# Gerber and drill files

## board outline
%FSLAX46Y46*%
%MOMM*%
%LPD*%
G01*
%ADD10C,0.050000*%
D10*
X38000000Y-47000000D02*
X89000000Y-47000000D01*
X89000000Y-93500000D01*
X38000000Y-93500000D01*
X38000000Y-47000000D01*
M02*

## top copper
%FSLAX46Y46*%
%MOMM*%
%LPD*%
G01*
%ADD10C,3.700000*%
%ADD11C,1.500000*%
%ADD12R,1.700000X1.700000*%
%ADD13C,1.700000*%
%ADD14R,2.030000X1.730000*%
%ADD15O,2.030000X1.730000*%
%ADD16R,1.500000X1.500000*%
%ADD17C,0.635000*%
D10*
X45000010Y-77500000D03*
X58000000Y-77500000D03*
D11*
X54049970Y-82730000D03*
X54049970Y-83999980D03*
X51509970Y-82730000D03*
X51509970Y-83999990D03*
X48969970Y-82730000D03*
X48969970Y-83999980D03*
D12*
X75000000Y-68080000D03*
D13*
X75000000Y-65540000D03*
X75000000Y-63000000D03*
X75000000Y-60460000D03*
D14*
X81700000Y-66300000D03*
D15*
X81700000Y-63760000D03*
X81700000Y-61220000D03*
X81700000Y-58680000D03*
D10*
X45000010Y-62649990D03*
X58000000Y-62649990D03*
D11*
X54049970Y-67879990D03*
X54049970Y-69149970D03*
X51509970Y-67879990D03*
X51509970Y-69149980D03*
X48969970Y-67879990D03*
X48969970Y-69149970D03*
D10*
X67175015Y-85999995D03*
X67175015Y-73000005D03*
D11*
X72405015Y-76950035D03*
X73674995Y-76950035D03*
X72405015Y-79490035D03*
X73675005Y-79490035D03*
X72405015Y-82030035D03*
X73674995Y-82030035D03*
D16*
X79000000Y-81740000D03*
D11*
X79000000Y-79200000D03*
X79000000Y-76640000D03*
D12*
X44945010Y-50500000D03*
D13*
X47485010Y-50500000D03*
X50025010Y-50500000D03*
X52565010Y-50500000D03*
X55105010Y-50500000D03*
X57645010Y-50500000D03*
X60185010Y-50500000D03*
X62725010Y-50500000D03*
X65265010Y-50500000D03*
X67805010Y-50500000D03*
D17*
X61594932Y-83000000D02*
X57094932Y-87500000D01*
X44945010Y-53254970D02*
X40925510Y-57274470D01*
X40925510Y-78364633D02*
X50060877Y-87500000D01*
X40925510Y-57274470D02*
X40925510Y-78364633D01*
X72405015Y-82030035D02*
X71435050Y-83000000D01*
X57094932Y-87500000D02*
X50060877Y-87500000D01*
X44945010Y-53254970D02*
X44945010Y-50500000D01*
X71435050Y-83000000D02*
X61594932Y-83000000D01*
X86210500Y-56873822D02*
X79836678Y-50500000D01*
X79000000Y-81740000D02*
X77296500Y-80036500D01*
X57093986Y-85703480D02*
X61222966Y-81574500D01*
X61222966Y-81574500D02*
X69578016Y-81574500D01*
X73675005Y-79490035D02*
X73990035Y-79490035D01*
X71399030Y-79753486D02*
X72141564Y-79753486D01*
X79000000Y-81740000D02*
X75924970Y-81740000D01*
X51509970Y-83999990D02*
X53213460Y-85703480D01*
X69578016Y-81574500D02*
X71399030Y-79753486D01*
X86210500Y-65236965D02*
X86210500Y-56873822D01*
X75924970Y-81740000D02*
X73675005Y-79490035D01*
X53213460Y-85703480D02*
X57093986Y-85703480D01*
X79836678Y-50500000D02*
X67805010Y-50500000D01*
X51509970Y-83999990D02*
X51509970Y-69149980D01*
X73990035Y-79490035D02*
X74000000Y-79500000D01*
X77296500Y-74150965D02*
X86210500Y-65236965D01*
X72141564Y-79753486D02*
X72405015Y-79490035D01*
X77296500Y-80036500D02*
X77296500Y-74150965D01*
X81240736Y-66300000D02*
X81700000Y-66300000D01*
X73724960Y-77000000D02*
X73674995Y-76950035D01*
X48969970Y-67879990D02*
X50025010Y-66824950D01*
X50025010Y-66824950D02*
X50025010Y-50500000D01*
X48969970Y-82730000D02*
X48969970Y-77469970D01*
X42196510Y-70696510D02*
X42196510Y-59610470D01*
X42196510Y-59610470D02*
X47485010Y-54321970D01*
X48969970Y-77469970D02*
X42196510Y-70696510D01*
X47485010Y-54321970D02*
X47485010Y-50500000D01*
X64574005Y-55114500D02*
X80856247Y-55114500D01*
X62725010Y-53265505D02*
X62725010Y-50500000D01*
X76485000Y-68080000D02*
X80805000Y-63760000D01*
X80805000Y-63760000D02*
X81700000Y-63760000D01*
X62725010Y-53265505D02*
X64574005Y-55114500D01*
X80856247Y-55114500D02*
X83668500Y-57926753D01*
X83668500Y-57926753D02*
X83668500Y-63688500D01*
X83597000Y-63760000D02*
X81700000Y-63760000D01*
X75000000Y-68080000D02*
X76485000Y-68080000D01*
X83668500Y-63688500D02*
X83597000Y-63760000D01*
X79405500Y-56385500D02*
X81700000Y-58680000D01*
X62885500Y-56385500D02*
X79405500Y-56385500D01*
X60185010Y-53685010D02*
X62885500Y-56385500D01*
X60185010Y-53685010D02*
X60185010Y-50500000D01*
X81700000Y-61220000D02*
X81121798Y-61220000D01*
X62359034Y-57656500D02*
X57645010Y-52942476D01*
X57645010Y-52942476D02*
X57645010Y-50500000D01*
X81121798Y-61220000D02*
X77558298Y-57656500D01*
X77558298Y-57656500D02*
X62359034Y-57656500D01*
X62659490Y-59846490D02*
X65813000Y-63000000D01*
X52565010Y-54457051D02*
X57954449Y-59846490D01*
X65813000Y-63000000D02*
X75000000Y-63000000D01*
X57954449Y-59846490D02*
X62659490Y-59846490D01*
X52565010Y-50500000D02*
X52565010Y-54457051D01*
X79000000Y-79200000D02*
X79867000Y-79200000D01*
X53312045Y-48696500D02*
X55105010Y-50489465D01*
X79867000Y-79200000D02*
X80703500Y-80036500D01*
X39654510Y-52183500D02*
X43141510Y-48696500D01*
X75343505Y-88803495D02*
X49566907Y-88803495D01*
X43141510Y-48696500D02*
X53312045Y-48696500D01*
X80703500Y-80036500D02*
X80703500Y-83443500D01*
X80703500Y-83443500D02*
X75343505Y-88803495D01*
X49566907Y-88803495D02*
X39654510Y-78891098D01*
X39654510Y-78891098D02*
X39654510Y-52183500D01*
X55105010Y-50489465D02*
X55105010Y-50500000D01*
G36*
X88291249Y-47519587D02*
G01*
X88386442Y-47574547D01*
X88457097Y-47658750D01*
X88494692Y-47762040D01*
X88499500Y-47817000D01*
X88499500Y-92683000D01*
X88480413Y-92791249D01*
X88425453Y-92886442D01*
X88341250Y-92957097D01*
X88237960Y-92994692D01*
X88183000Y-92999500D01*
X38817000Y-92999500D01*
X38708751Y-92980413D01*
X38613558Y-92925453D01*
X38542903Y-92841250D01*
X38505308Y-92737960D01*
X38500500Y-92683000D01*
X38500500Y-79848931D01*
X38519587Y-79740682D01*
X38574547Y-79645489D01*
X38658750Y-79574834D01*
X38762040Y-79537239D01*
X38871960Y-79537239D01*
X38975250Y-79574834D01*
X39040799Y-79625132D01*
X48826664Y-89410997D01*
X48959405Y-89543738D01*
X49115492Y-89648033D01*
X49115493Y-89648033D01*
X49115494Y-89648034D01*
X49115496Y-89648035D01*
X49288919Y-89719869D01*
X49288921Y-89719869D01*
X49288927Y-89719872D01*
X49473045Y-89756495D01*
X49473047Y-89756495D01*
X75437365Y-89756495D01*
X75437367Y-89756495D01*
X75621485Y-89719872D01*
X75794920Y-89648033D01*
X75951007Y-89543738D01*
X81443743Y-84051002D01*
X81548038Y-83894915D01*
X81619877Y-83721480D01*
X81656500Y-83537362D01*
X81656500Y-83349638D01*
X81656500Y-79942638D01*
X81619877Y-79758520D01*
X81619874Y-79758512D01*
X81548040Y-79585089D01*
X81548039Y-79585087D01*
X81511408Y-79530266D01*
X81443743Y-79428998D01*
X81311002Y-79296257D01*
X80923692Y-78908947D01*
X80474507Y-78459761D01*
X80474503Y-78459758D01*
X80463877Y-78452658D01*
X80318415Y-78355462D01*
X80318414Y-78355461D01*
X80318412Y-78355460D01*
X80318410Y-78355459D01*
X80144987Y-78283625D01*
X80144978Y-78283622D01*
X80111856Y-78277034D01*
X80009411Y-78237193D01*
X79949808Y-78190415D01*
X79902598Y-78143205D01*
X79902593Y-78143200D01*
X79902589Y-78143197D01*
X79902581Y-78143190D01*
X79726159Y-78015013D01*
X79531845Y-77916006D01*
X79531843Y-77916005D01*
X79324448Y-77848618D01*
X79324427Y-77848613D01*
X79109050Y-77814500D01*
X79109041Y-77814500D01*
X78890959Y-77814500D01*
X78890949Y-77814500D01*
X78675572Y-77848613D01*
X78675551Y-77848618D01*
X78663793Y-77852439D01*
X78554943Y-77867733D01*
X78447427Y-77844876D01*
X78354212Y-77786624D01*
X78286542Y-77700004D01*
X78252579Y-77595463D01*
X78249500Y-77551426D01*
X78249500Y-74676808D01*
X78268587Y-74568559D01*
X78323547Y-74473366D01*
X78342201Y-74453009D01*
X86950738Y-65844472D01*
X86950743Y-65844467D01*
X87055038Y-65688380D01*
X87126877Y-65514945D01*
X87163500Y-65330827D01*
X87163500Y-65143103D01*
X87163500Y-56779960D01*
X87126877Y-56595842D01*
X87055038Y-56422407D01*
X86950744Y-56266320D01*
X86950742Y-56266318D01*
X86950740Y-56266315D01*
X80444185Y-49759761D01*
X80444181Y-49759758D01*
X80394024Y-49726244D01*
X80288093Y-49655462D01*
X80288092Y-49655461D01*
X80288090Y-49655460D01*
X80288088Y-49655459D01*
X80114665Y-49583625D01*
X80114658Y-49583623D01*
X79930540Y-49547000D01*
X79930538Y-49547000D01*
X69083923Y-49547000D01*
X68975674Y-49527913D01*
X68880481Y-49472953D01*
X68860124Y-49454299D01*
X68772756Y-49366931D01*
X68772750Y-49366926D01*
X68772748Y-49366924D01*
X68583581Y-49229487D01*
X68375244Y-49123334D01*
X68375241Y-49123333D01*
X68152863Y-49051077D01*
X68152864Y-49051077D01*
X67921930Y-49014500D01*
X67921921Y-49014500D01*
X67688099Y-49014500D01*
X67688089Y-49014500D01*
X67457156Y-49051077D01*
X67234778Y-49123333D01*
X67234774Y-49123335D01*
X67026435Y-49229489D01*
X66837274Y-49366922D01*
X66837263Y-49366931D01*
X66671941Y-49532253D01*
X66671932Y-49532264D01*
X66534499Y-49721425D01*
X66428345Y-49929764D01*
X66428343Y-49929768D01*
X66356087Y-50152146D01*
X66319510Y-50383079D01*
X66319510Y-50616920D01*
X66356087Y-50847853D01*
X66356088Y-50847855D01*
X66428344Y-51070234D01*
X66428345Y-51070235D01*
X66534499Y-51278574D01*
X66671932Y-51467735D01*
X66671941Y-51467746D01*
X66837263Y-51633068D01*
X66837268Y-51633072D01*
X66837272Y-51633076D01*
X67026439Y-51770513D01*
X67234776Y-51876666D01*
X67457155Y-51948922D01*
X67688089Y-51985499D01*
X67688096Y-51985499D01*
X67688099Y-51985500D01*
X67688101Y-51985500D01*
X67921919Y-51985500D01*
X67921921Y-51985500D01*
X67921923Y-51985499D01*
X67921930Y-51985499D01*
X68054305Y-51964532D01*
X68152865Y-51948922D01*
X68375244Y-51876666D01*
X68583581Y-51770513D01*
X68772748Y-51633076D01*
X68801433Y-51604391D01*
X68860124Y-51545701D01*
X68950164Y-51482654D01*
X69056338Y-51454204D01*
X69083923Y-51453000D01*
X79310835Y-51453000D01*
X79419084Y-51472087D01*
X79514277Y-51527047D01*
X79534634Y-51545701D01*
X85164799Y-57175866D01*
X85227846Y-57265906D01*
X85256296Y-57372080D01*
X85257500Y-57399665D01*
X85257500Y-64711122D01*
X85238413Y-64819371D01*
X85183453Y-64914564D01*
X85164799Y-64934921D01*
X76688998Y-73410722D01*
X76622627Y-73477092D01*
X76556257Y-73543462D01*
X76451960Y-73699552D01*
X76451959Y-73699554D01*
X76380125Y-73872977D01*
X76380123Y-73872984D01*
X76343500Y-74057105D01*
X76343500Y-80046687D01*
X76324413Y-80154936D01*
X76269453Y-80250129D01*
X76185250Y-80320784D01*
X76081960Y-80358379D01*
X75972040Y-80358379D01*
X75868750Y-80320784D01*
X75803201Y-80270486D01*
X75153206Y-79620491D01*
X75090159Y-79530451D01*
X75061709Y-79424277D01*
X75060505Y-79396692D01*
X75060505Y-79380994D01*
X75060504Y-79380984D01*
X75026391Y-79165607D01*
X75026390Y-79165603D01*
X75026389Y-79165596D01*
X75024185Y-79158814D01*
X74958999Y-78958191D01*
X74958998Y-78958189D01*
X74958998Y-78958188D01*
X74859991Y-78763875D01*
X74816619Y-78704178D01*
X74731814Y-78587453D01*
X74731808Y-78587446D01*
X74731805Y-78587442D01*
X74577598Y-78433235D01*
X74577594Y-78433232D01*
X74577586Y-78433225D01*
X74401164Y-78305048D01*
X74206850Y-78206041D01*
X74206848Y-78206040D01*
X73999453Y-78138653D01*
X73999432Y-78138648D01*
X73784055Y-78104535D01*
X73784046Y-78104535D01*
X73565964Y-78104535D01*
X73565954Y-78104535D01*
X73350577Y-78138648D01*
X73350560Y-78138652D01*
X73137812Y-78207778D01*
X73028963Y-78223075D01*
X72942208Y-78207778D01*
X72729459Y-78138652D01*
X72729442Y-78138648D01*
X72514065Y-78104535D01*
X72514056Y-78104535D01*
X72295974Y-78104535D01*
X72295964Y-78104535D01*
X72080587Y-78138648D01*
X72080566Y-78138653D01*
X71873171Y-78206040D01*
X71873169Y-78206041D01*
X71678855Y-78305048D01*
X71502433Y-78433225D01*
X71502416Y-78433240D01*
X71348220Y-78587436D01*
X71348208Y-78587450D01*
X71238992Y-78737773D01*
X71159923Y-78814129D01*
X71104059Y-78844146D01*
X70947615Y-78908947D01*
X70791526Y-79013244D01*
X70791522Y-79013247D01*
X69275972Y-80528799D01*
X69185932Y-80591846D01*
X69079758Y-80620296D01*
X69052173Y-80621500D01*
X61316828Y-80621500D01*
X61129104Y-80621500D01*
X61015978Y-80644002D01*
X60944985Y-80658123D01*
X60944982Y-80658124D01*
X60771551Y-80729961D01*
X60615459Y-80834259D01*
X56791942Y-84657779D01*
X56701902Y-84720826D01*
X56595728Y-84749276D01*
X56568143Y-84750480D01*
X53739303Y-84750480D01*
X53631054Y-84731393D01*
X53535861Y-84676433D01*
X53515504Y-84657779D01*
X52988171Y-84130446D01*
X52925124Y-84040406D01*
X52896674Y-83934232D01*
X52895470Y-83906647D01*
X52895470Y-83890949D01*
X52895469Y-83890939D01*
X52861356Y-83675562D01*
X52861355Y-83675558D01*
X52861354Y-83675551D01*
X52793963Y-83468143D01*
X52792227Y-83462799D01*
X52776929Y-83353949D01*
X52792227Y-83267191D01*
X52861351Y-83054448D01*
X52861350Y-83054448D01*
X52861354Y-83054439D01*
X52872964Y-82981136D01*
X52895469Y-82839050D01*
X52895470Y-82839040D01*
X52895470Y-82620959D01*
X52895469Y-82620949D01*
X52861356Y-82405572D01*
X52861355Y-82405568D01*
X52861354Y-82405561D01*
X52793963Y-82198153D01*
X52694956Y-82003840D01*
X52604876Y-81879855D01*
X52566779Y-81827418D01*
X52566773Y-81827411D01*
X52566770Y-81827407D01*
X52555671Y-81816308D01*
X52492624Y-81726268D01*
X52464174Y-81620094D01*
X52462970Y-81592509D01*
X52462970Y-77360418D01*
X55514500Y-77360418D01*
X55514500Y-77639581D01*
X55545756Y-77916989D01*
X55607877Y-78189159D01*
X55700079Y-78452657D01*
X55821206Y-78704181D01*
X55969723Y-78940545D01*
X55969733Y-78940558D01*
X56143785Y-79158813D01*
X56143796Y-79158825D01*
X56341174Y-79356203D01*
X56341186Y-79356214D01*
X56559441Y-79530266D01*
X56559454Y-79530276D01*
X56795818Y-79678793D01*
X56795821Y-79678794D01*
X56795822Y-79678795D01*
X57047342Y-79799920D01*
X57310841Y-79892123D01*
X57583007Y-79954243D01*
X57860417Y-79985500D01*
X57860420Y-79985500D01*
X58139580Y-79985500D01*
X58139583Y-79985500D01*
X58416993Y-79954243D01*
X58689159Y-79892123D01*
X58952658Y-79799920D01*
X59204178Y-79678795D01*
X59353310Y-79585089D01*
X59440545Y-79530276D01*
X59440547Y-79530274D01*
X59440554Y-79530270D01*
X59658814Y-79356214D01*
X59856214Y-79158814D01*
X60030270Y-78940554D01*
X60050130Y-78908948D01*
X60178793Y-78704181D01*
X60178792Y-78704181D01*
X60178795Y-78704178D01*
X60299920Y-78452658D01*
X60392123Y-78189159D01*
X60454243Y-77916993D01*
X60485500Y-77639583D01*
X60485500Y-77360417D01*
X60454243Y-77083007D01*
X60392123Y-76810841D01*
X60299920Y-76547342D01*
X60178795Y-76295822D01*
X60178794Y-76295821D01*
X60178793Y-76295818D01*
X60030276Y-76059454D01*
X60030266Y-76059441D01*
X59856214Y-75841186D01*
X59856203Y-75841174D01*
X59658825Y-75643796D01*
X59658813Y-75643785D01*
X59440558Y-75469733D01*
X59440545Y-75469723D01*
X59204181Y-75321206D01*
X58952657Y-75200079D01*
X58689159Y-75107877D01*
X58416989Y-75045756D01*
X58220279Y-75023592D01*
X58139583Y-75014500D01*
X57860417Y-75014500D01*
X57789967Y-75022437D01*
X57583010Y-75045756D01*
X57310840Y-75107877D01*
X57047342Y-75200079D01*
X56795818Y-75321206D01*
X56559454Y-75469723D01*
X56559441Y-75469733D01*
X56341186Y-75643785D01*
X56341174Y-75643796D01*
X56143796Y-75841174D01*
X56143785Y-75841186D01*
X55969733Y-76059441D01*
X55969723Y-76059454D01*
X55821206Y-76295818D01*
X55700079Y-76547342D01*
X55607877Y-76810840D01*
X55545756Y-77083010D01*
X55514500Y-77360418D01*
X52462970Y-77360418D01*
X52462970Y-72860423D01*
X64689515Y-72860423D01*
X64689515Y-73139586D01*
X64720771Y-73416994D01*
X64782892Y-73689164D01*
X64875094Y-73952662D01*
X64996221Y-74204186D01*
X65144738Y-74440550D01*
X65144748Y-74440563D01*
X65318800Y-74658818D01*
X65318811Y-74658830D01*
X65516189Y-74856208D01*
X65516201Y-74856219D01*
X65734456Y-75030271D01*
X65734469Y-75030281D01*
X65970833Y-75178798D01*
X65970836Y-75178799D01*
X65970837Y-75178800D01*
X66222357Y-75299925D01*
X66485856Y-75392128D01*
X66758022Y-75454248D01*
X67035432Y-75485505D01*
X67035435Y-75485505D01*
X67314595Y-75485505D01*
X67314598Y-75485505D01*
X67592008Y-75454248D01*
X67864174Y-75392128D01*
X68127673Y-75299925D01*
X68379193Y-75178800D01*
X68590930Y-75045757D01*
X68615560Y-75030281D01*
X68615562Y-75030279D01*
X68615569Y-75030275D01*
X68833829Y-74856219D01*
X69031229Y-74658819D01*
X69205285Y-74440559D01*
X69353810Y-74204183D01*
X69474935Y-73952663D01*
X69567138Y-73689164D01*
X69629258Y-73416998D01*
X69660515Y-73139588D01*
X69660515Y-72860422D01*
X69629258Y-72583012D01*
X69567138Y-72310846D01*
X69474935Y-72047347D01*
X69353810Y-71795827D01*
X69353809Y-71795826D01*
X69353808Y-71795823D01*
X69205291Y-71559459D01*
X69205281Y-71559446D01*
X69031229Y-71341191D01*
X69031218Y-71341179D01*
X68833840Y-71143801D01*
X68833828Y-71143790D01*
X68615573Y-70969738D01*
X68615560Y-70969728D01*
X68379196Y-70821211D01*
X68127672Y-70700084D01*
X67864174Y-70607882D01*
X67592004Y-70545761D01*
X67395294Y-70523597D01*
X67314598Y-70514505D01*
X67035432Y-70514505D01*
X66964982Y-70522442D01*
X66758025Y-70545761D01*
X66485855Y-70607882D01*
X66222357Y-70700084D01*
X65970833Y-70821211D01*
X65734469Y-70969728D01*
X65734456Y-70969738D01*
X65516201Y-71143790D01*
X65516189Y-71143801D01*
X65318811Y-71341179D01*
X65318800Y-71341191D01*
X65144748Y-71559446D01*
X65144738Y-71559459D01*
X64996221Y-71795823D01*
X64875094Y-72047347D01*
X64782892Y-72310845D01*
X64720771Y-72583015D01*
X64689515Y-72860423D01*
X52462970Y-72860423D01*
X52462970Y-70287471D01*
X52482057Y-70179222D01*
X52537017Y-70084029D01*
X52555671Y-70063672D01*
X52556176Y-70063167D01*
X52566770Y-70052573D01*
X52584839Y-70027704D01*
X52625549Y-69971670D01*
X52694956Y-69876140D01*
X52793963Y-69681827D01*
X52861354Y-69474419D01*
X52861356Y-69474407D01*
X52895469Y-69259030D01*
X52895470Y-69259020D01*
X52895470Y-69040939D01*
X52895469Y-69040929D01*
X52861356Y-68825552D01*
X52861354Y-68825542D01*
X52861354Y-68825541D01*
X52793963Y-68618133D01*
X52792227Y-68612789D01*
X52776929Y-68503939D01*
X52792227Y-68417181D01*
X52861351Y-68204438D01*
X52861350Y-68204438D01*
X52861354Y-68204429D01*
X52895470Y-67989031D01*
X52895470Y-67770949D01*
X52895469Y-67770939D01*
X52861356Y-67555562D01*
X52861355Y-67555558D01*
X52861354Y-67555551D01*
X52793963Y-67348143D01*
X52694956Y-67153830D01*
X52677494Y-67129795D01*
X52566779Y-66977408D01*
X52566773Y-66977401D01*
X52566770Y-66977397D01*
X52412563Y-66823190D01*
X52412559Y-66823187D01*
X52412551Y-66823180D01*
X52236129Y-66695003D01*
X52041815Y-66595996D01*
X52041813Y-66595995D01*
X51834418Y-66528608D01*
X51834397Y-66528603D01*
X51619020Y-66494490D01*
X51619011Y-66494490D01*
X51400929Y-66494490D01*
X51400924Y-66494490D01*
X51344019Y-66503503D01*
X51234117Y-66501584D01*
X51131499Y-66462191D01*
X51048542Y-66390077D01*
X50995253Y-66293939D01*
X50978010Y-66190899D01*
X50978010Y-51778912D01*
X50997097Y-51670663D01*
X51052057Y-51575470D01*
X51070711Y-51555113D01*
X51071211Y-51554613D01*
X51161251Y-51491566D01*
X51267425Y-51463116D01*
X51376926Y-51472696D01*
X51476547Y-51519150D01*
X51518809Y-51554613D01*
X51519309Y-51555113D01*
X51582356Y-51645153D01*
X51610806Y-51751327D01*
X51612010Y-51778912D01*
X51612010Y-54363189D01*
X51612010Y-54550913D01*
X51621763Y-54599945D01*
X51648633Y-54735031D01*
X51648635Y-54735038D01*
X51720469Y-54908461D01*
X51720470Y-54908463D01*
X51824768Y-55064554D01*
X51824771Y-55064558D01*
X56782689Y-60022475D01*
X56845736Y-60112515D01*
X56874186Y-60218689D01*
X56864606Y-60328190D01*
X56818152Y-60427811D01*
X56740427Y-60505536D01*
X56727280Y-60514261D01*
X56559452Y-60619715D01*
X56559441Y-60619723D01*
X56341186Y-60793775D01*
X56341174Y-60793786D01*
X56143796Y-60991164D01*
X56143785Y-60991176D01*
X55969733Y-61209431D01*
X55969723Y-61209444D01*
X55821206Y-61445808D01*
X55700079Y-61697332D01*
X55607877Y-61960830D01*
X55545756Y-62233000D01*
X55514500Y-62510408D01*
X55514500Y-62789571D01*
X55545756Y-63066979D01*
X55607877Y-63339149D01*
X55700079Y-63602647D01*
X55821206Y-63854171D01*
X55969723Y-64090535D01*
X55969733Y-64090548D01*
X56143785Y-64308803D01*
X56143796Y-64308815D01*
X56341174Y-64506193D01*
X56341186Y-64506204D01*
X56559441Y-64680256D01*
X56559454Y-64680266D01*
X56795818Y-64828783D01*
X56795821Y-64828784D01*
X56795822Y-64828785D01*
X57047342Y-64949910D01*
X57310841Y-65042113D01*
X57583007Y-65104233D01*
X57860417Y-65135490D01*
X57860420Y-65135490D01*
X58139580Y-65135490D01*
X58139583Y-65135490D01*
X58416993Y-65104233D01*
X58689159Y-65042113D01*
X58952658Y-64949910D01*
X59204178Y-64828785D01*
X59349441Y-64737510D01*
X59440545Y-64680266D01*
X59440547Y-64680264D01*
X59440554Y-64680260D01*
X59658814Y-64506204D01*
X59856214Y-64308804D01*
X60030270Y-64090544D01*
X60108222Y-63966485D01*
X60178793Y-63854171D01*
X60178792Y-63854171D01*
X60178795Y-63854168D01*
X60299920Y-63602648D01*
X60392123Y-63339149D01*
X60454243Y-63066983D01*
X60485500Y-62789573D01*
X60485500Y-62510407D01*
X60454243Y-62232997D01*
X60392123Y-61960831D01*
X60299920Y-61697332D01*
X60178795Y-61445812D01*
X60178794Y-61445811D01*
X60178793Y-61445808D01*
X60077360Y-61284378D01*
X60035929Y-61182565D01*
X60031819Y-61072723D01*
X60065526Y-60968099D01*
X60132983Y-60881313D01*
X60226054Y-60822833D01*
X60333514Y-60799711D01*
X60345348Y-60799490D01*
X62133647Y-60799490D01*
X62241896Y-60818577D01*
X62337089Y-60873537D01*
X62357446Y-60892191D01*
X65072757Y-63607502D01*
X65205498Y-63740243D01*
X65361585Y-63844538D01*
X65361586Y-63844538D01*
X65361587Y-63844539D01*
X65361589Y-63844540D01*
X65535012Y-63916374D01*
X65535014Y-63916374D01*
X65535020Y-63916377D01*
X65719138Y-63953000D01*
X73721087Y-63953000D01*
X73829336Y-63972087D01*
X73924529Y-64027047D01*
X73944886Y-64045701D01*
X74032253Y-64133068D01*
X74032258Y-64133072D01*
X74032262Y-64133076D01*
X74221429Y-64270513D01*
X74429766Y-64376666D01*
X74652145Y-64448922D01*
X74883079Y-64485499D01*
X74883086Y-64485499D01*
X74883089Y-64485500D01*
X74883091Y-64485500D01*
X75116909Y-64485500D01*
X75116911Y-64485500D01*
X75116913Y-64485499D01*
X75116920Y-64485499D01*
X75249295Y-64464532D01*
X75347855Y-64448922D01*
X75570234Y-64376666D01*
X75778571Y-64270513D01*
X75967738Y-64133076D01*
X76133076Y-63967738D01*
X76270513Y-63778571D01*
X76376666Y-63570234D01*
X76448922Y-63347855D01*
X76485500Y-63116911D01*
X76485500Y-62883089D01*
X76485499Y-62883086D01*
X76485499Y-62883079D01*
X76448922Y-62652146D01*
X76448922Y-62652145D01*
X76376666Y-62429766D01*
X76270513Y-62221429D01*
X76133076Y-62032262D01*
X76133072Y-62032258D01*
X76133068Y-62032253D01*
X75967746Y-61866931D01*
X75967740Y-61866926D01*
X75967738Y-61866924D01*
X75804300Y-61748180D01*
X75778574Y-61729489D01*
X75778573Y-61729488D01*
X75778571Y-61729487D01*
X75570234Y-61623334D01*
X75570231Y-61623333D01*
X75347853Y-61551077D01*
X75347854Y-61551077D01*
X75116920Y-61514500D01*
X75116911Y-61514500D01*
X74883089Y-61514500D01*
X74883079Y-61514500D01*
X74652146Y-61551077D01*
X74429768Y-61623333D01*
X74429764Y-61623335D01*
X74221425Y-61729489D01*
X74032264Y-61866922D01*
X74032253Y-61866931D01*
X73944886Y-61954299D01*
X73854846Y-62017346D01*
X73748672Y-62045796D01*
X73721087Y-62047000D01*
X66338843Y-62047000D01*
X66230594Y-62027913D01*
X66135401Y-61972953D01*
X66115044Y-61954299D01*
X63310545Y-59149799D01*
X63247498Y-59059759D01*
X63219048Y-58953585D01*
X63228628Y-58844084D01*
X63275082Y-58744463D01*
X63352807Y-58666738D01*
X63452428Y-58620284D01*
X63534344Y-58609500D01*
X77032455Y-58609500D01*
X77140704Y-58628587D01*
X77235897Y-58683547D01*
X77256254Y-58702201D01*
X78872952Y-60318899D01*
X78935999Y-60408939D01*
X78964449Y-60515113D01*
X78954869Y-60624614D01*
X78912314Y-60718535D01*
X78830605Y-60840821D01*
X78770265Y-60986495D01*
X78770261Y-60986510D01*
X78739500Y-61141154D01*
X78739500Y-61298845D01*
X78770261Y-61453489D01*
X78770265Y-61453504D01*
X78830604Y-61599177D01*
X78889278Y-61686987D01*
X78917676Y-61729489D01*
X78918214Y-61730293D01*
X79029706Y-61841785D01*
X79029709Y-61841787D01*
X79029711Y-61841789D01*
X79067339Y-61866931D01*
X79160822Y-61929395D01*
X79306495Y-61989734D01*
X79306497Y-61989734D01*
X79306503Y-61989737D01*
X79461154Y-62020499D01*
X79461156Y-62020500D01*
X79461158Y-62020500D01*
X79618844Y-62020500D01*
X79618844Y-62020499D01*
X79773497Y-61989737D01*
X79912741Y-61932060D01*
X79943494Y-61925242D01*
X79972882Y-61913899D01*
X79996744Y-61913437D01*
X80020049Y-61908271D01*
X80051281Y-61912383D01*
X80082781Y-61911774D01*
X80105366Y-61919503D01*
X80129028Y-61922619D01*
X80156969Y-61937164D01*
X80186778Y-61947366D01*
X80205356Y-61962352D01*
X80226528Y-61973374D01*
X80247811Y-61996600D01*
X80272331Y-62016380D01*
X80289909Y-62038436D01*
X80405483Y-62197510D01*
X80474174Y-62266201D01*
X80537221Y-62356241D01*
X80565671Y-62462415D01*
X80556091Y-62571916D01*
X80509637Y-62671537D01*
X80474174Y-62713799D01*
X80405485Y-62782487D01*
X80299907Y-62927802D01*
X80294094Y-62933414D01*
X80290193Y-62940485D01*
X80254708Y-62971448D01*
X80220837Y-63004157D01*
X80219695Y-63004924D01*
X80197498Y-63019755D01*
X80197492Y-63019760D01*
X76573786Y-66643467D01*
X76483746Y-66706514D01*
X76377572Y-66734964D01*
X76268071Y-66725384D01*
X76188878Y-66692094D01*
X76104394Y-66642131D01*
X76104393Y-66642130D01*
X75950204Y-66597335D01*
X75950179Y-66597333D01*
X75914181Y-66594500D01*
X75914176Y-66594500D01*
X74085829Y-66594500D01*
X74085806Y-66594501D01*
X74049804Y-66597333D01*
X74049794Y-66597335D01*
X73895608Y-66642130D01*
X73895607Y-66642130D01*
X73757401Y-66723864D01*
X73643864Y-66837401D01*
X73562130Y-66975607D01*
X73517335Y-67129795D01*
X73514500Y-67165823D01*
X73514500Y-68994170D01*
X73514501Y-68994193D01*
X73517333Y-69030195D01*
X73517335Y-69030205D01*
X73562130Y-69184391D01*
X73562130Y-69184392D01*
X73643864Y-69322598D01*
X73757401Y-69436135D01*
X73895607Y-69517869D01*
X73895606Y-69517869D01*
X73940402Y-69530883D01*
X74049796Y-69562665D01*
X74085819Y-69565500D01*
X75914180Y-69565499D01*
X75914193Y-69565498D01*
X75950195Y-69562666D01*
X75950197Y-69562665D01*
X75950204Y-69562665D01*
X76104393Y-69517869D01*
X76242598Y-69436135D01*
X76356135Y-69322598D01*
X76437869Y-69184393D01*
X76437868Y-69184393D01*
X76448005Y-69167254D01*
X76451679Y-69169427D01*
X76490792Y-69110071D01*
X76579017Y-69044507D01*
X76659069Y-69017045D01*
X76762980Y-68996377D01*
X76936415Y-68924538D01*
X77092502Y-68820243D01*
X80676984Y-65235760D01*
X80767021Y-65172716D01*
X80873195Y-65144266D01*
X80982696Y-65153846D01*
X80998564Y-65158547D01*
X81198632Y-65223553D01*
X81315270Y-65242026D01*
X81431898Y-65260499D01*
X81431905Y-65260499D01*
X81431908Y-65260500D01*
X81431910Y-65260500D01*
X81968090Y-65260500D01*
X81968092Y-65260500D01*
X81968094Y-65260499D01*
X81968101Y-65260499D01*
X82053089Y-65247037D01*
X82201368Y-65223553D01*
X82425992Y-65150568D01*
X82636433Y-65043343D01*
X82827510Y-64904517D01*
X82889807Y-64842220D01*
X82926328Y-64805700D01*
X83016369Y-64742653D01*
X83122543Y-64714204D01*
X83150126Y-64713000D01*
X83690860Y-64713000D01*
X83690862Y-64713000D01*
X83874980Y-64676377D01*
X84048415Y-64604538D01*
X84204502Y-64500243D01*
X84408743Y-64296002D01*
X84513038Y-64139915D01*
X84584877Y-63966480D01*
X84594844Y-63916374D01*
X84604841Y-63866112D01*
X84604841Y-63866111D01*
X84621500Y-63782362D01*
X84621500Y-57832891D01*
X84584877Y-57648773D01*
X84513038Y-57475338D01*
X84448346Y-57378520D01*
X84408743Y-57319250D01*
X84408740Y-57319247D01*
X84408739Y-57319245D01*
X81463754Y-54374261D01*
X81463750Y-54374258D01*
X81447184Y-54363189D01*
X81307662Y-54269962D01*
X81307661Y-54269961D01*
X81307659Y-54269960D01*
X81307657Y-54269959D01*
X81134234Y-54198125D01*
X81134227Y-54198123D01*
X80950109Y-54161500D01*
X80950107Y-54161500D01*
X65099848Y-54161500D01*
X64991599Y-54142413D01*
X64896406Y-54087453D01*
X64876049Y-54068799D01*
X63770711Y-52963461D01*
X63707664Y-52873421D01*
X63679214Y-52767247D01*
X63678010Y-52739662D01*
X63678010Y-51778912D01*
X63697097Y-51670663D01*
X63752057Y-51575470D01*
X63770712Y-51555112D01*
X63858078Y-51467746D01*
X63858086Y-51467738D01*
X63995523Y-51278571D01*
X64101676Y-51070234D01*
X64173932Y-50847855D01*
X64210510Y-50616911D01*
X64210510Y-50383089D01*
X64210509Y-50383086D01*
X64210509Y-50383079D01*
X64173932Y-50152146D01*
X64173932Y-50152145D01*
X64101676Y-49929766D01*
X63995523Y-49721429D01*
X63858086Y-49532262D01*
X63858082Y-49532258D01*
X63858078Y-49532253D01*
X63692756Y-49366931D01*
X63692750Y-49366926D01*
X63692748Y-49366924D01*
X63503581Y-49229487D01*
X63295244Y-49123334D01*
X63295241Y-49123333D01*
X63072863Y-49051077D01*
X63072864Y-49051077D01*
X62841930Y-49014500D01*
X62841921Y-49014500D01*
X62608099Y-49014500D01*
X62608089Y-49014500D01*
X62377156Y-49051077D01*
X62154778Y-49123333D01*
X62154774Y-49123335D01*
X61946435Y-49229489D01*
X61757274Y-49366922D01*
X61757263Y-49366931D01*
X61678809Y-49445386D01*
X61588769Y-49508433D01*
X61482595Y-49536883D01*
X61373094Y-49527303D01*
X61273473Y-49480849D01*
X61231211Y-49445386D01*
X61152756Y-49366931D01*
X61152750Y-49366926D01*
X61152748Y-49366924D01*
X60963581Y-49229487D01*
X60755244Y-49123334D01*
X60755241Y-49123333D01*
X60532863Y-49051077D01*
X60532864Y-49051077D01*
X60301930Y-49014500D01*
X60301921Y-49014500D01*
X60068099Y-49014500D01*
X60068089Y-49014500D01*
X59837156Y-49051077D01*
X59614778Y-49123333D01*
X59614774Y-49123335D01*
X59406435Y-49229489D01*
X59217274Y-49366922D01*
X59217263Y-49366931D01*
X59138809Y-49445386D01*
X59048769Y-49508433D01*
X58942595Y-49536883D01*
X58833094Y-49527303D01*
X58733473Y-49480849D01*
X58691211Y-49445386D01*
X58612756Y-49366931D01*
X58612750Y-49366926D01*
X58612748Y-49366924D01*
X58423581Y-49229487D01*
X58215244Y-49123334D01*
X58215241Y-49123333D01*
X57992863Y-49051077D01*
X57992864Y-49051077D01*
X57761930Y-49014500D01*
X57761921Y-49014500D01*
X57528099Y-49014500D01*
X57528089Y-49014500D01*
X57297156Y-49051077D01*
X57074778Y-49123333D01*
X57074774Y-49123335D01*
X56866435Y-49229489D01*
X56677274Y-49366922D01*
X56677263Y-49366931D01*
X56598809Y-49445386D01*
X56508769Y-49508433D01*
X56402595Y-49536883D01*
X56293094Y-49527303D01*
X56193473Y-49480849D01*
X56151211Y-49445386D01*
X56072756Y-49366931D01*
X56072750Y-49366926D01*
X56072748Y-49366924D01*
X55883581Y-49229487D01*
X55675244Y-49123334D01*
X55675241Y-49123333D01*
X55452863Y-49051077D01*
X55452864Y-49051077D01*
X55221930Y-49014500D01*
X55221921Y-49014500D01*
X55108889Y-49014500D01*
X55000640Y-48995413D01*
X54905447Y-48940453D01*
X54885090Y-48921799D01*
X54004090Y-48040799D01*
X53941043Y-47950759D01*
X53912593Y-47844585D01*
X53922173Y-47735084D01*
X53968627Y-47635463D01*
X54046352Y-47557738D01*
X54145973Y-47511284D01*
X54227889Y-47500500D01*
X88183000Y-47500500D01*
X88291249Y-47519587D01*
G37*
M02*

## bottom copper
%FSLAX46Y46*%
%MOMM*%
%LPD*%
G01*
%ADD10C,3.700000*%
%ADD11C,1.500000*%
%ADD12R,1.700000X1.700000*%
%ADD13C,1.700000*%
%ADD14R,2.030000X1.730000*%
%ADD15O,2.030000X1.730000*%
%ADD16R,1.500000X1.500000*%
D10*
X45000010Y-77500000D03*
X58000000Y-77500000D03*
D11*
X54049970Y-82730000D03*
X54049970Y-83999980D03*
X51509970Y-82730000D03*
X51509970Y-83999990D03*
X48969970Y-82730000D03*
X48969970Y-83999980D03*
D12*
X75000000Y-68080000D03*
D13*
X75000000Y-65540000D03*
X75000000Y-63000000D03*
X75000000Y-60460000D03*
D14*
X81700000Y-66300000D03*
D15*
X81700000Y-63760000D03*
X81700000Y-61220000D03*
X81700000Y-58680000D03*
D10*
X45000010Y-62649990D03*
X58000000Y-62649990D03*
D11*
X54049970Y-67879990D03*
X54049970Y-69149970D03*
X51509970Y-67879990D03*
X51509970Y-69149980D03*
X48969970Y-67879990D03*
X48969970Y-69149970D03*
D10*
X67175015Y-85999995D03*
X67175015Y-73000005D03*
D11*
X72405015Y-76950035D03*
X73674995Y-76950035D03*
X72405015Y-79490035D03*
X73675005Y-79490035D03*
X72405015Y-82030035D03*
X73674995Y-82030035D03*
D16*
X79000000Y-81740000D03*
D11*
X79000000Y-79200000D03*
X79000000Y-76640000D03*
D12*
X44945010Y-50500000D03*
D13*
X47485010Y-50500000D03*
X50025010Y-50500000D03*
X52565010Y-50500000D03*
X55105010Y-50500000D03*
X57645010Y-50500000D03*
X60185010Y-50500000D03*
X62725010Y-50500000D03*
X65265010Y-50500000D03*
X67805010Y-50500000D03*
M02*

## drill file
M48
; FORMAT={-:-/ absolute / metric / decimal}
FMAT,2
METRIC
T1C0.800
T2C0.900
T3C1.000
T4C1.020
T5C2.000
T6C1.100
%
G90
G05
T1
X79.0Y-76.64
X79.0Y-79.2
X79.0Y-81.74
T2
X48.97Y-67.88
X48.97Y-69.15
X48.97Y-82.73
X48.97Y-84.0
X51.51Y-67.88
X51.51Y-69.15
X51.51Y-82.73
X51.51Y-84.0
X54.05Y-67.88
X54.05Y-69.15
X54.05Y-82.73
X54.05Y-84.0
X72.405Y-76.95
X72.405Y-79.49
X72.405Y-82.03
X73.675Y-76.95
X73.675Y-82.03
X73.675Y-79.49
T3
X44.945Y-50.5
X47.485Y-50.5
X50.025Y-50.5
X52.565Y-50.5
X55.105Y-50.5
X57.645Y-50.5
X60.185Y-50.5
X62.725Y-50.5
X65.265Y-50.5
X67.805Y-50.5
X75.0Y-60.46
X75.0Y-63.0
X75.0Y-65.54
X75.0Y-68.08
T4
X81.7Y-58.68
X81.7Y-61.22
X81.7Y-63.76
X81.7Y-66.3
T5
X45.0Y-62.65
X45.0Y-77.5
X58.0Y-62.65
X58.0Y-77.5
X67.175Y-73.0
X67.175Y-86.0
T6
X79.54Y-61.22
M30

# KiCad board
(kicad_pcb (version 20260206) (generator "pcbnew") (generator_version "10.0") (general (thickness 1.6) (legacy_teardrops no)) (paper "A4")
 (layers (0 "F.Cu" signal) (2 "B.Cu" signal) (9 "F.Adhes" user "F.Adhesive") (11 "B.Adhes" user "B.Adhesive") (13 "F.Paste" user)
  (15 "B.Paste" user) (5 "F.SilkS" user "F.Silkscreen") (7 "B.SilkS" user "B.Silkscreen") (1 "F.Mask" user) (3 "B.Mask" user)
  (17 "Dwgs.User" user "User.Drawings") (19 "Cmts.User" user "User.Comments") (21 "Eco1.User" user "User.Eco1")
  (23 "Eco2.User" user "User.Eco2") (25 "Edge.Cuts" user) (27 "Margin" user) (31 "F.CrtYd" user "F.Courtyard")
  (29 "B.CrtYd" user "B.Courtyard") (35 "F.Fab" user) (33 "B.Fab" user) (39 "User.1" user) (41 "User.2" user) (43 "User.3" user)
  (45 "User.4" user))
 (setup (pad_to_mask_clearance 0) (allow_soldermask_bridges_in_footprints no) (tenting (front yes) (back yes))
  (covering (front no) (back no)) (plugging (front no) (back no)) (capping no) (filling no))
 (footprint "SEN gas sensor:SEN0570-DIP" (layer "F.Cu") (at 45.00001 77.5)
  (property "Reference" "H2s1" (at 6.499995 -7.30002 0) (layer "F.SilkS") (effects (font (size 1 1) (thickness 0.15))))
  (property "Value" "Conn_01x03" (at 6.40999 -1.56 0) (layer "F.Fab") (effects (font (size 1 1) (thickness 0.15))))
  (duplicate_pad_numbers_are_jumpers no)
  (pad "0" thru_hole circle (at 0 0 180) (size 3.7 3.7) (drill 2) (layers "*.Cu" "*.Mask") (remove_unused_layers no)
   (solder_paste_margin -111) (thermal_bridge_angle 90))
  (pad "0" thru_hole circle (at 12.99999 0 180) (size 3.7 3.7) (drill 2) (layers "*.Cu" "*.Mask") (remove_unused_layers no)
   (solder_paste_margin -111) (thermal_bridge_angle 90))
  (pad "1" thru_hole circle (at 9.04996 5.23 180) (size 1.5 1.5) (drill 0.9) (layers "*.Cu" "*.Mask") (remove_unused_layers no) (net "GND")
   (thermal_bridge_angle 90))
  (pad "1" thru_hole circle (at 9.04996 6.49998 180) (size 1.5 1.5) (drill 0.9) (layers "*.Cu" "*.Mask") (remove_unused_layers no)
   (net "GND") (thermal_bridge_angle 90))
  (pad "2" thru_hole circle (at 6.50996 5.23 180) (size 1.5 1.5) (drill 0.9) (layers "*.Cu" "*.Mask") (remove_unused_layers no)
   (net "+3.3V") (thermal_bridge_angle 90))
  (pad "2" thru_hole circle (at 6.50996 6.49999 180) (size 1.5 1.5) (drill 0.9) (layers "*.Cu" "*.Mask") (remove_unused_layers no)
   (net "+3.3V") (thermal_bridge_angle 90))
  (pad "3" thru_hole circle (at 3.96996 5.23 180) (size 1.5 1.5) (drill 0.9) (layers "*.Cu" "*.Mask") (remove_unused_layers no) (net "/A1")
   (thermal_bridge_angle 90))
  (pad "3" thru_hole circle (at 3.96996 6.49998 180) (size 1.5 1.5) (drill 0.9) (layers "*.Cu" "*.Mask") (remove_unused_layers no)
   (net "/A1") (thermal_bridge_angle 90)))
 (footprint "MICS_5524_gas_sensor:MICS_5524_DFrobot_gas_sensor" (layer "F.Cu") (at 68 65 90)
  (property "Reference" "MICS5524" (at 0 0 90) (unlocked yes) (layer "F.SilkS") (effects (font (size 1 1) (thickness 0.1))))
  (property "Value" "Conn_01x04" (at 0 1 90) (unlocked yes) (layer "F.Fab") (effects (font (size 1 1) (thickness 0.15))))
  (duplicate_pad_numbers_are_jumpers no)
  (pad "1" thru_hole rect (at -3.08 7 180) (size 1.7 1.7) (drill 1) (layers "*.Cu" "*.Mask") (remove_unused_layers no) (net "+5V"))
  (pad "2" thru_hole circle (at -0.54 7 180) (size 1.7 1.7) (drill 1) (layers "*.Cu" "*.Mask") (remove_unused_layers no) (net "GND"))
  (pad "3" thru_hole circle (at 2 7 180) (size 1.7 1.7) (drill 1) (layers "*.Cu" "*.Mask") (remove_unused_layers no) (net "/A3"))
  (pad "4" thru_hole circle (at 4.54 7 180) (size 1.7 1.7) (drill 1) (layers "*.Cu" "*.Mask") (remove_unused_layers no) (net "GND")))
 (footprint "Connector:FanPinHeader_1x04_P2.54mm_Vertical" (layer "F.Cu") (at 81.7 66.3 90)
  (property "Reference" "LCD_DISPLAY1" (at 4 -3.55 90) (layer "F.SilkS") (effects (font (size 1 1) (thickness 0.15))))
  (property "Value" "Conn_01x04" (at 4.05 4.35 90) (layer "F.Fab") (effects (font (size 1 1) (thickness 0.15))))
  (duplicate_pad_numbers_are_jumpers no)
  (pad "" np_thru_hole circle (at 5.08 -2.16 180) (size 1.1 1.1) (drill 1.1) (layers "*.Cu" "*.Mask"))
  (pad "1" thru_hole rect (at 0 0 180) (size 2.03 1.73) (drill 1.02) (layers "*.Cu" "*.Mask") (remove_unused_layers no) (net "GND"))
  (pad "2" thru_hole oval (at 2.54 0 180) (size 2.03 1.73) (drill 1.02) (layers "*.Cu" "*.Mask") (remove_unused_layers no) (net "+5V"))
  (pad "3" thru_hole oval (at 5.08 0 180) (size 2.03 1.73) (drill 1.02) (layers "*.Cu" "*.Mask") (remove_unused_layers no) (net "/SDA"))
  (pad "4" thru_hole oval (at 7.62 0 180) (size 2.03 1.73) (drill 1.02) (layers "*.Cu" "*.Mask") (remove_unused_layers no) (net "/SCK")))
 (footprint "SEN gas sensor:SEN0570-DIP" (layer "F.Cu") (at 45.00001 62.64999)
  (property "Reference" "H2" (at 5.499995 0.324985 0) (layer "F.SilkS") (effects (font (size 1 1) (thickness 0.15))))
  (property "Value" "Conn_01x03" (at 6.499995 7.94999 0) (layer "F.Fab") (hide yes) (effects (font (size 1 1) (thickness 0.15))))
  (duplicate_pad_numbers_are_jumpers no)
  (pad "0" thru_hole circle (at 0 0 180) (size 3.7 3.7) (drill 2) (layers "*.Cu" "*.Mask") (remove_unused_layers no)
   (solder_paste_margin -111) (thermal_bridge_angle 90))
  (pad "0" thru_hole circle (at 12.99999 0 180) (size 3.7 3.7) (drill 2) (layers "*.Cu" "*.Mask") (remove_unused_layers no)
   (solder_paste_margin -111) (thermal_bridge_angle 90))
  (pad "1" thru_hole circle (at 9.04996 5.23 180) (size 1.5 1.5) (drill 0.9) (layers "*.Cu" "*.Mask") (remove_unused_layers no) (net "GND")
   (thermal_bridge_angle 90))
  (pad "1" thru_hole circle (at 9.04996 6.49998 180) (size 1.5 1.5) (drill 0.9) (layers "*.Cu" "*.Mask") (remove_unused_layers no)
   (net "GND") (thermal_bridge_angle 90))
  (pad "2" thru_hole circle (at 6.50996 5.23 180) (size 1.5 1.5) (drill 0.9) (layers "*.Cu" "*.Mask") (remove_unused_layers no)
   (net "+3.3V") (thermal_bridge_angle 90))
  (pad "2" thru_hole circle (at 6.50996 6.49999 180) (size 1.5 1.5) (drill 0.9) (layers "*.Cu" "*.Mask") (remove_unused_layers no)
   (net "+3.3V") (thermal_bridge_angle 90))
  (pad "3" thru_hole circle (at 3.96996 5.23 180) (size 1.5 1.5) (drill 0.9) (layers "*.Cu" "*.Mask") (remove_unused_layers no) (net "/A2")
   (thermal_bridge_angle 90))
  (pad "3" thru_hole circle (at 3.96996 6.49998 180) (size 1.5 1.5) (drill 0.9) (layers "*.Cu" "*.Mask") (remove_unused_layers no)
   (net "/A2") (thermal_bridge_angle 90)))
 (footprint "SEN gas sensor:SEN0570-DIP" (layer "F.Cu") (at 67.175015 85.999995 90)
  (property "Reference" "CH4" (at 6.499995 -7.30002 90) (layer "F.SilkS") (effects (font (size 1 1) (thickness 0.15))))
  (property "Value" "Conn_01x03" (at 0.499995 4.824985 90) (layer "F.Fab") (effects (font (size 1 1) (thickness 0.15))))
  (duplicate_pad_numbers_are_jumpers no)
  (pad "0" thru_hole circle (at 0 0 270) (size 3.7 3.7) (drill 2) (layers "*.Cu" "*.Mask") (remove_unused_layers no)
   (solder_paste_margin -111) (thermal_bridge_angle 90))
  (pad "0" thru_hole circle (at 12.99999 0 270) (size 3.7 3.7) (drill 2) (layers "*.Cu" "*.Mask") (remove_unused_layers no)
   (solder_paste_margin -111) (thermal_bridge_angle 90))
  (pad "1" thru_hole circle (at 9.04996 5.23 270) (size 1.5 1.5) (drill 0.9) (layers "*.Cu" "*.Mask") (remove_unused_layers no) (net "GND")
   (thermal_bridge_angle 90))
  (pad "1" thru_hole circle (at 9.04996 6.49998 270) (size 1.5 1.5) (drill 0.9) (layers "*.Cu" "*.Mask") (remove_unused_layers no)
   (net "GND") (thermal_bridge_angle 90))
  (pad "2" thru_hole circle (at 6.50996 5.23 270) (size 1.5 1.5) (drill 0.9) (layers "*.Cu" "*.Mask") (remove_unused_layers no)
   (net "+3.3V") (thermal_bridge_angle 90))
  (pad "2" thru_hole circle (at 6.50996 6.49999 270) (size 1.5 1.5) (drill 0.9) (layers "*.Cu" "*.Mask") (remove_unused_layers no)
   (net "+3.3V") (thermal_bridge_angle 90))
  (pad "3" thru_hole circle (at 3.96996 5.23 270) (size 1.5 1.5) (drill 0.9) (layers "*.Cu" "*.Mask") (remove_unused_layers no) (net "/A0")
   (thermal_bridge_angle 90))
  (pad "3" thru_hole circle (at 3.96996 6.49998 270) (size 1.5 1.5) (drill 0.9) (layers "*.Cu" "*.Mask") (remove_unused_layers no)
   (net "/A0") (thermal_bridge_angle 90)))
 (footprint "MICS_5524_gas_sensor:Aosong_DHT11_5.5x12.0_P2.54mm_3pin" (layer "F.Cu") (at 79 83 180)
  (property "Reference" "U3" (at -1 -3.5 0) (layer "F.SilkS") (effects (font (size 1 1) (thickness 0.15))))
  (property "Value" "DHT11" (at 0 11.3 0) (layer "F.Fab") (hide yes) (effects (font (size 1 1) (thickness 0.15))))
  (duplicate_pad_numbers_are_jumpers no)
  (pad "1" thru_hole rect (at 0 1.26 180) (size 1.5 1.5) (drill 0.8) (layers "*.Cu" "*.Mask") (remove_unused_layers no) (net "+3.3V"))
  (pad "2" thru_hole circle (at 0 3.8 180) (size 1.5 1.5) (drill 0.8) (layers "*.Cu" "*.Mask") (remove_unused_layers no) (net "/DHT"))
  (pad "4" thru_hole circle (at 0 6.36 180) (size 1.5 1.5) (drill 0.8) (layers "*.Cu" "*.Mask") (remove_unused_layers no) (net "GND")))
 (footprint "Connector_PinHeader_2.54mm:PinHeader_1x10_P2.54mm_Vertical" (layer "F.Cu") (at 44.94501 50.5 90)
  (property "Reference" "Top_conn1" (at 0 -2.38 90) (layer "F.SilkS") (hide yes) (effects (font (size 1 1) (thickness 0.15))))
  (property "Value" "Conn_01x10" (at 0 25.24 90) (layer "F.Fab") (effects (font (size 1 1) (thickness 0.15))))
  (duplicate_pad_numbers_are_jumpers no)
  (pad "1" thru_hole rect (at 0 0 90) (size 1.7 1.7) (drill 1) (layers "*.Cu" "*.Mask") (remove_unused_layers no) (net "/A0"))
  (pad "2" thru_hole circle (at 0 2.54 90) (size 1.7 1.7) (drill 1) (layers "*.Cu" "*.Mask") (remove_unused_layers no) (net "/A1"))
  (pad "3" thru_hole circle (at 0 5.08 90) (size 1.7 1.7) (drill 1) (layers "*.Cu" "*.Mask") (remove_unused_layers no) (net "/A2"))
  (pad "4" thru_hole circle (at 0 7.62 90) (size 1.7 1.7) (drill 1) (layers "*.Cu" "*.Mask") (remove_unused_layers no) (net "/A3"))
  (pad "5" thru_hole circle (at 0 10.16 90) (size 1.7 1.7) (drill 1) (layers "*.Cu" "*.Mask") (remove_unused_layers no) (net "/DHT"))
  (pad "6" thru_hole circle (at 0 12.7 90) (size 1.7 1.7) (drill 1) (layers "*.Cu" "*.Mask") (remove_unused_layers no) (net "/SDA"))
  (pad "7" thru_hole circle (at 0 15.24 90) (size 1.7 1.7) (drill 1) (layers "*.Cu" "*.Mask") (remove_unused_layers no) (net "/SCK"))
  (pad "8" thru_hole circle (at 0 17.78 90) (size 1.7 1.7) (drill 1) (layers "*.Cu" "*.Mask") (remove_unused_layers no) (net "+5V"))
  (pad "9" thru_hole circle (at 0 20.32 90) (size 1.7 1.7) (drill 1) (layers "*.Cu" "*.Mask") (remove_unused_layers no) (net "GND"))
  (pad "10" thru_hole circle (at 0 22.86 90) (size 1.7 1.7) (drill 1) (layers "*.Cu" "*.Mask") (remove_unused_layers no) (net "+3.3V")))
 (gr_rect (start 38 47) (end 89 93.5) (stroke (width 0.05) (type default)) (fill no) (layer "Edge.Cuts"))
 (segment (start 61.594932 83) (end 57.094932 87.5) (width 0.635) (layer "F.Cu") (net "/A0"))
 (segment (start 44.94501 53.25497) (end 40.92551 57.27447) (width 0.635) (layer "F.Cu") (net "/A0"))
 (segment (start 40.92551 78.364633) (end 50.060877 87.5) (width 0.635) (layer "F.Cu") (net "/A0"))
 (segment (start 40.92551 57.27447) (end 40.92551 78.364633) (width 0.635) (layer "F.Cu") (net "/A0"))
 (segment (start 72.405015 82.030035) (end 71.43505 83) (width 0.635) (layer "F.Cu") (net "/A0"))
 (segment (start 57.094932 87.5) (end 50.060877 87.5) (width 0.635) (layer "F.Cu") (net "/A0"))
 (segment (start 44.94501 53.25497) (end 44.94501 50.5) (width 0.635) (layer "F.Cu") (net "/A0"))
 (segment (start 71.43505 83) (end 61.594932 83) (width 0.635) (layer "F.Cu") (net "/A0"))
 (segment (start 86.2105 56.873822) (end 79.836678 50.5) (width 0.635) (layer "F.Cu") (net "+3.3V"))
 (segment (start 79 81.74) (end 77.2965 80.0365) (width 0.635) (layer "F.Cu") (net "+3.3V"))
 (segment (start 57.093986 85.70348) (end 61.222966 81.5745) (width 0.635) (layer "F.Cu") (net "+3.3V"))
 (segment (start 61.222966 81.5745) (end 69.578016 81.5745) (width 0.635) (layer "F.Cu") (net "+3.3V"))
 (segment (start 73.675005 79.490035) (end 73.990035 79.490035) (width 0.635) (layer "F.Cu") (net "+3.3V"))
 (segment (start 71.39903 79.753486) (end 72.141564 79.753486) (width 0.635) (layer "F.Cu") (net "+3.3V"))
 (segment (start 79 81.74) (end 75.92497 81.74) (width 0.635) (layer "F.Cu") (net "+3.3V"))
 (segment (start 51.50997 83.99999) (end 53.21346 85.70348) (width 0.635) (layer "F.Cu") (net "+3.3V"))
 (segment (start 69.578016 81.5745) (end 71.39903 79.753486) (width 0.635) (layer "F.Cu") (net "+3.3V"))
 (segment (start 86.2105 65.236965) (end 86.2105 56.873822) (width 0.635) (layer "F.Cu") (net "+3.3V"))
 (segment (start 75.92497 81.74) (end 73.675005 79.490035) (width 0.635) (layer "F.Cu") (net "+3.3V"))
 (segment (start 53.21346 85.70348) (end 57.093986 85.70348) (width 0.635) (layer "F.Cu") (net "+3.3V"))
 (segment (start 79.836678 50.5) (end 67.80501 50.5) (width 0.635) (layer "F.Cu") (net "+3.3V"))
 (segment (start 51.50997 83.99999) (end 51.50997 69.14998) (width 0.635) (layer "F.Cu") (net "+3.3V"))
 (segment (start 73.990035 79.490035) (end 74 79.5) (width 0.635) (layer "F.Cu") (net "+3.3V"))
 (segment (start 77.2965 74.150965) (end 86.2105 65.236965) (width 0.635) (layer "F.Cu") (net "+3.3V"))
 (segment (start 72.141564 79.753486) (end 72.405015 79.490035) (width 0.635) (layer "F.Cu") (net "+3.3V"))
 (segment (start 77.2965 80.0365) (end 77.2965 74.150965) (width 0.635) (layer "F.Cu") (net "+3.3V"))
 (segment (start 81.240736 66.3) (end 81.7 66.3) (width 0.635) (layer "F.Cu") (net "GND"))
 (segment (start 73.72496 77) (end 73.674995 76.950035) (width 0.635) (layer "F.Cu") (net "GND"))
 (segment (start 48.96997 67.87999) (end 50.02501 66.82495) (width 0.635) (layer "F.Cu") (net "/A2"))
 (segment (start 50.02501 66.82495) (end 50.02501 50.5) (width 0.635) (layer "F.Cu") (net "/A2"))
 (segment (start 48.96997 82.73) (end 48.96997 77.46997) (width 0.635) (layer "F.Cu") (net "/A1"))
 (segment (start 42.19651 70.69651) (end 42.19651 59.61047) (width 0.635) (layer "F.Cu") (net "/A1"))
 (segment (start 42.19651 59.61047) (end 47.48501 54.32197) (width 0.635) (layer "F.Cu") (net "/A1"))
 (segment (start 48.96997 77.46997) (end 42.19651 70.69651) (width 0.635) (layer "F.Cu") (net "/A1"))
 (segment (start 47.48501 54.32197) (end 47.48501 50.5) (width 0.635) (layer "F.Cu") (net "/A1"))
 (segment (start 64.574005 55.1145) (end 80.856247 55.1145) (width 0.635) (layer "F.Cu") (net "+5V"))
 (segment (start 62.72501 53.265505) (end 62.72501 50.5) (width 0.635) (layer "F.Cu") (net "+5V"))
 (segment (start 76.485 68.08) (end 80.805 63.76) (width 0.635) (layer "F.Cu") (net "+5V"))
 (segment (start 80.805 63.76) (end 81.7 63.76) (width 0.635) (layer "F.Cu") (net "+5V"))
 (segment (start 62.72501 53.265505) (end 64.574005 55.1145) (width 0.635) (layer "F.Cu") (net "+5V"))
 (segment (start 80.856247 55.1145) (end 83.6685 57.926753) (width 0.635) (layer "F.Cu") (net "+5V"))
 (segment (start 83.6685 57.926753) (end 83.6685 63.6885) (width 0.635) (layer "F.Cu") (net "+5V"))
 (segment (start 83.597 63.76) (end 81.7 63.76) (width 0.635) (layer "F.Cu") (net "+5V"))
 (segment (start 75 68.08) (end 76.485 68.08) (width 0.635) (layer "F.Cu") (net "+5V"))
 (segment (start 83.6685 63.6885) (end 83.597 63.76) (width 0.635) (layer "F.Cu") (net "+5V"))
 (segment (start 79.4055 56.3855) (end 81.7 58.68) (width 0.635) (layer "F.Cu") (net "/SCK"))
 (segment (start 62.8855 56.3855) (end 79.4055 56.3855) (width 0.635) (layer "F.Cu") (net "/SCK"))
 (segment (start 60.18501 53.68501) (end 62.8855 56.3855) (width 0.635) (layer "F.Cu") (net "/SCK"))
 (segment (start 60.18501 53.68501) (end 60.18501 50.5) (width 0.635) (layer "F.Cu") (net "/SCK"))
 (segment (start 81.7 61.22) (end 81.121798 61.22) (width 0.635) (layer "F.Cu") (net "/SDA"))
 (segment (start 62.359034 57.6565) (end 57.64501 52.942476) (width 0.635) (layer "F.Cu") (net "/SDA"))
 (segment (start 57.64501 52.942476) (end 57.64501 50.5) (width 0.635) (layer "F.Cu") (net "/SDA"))
 (segment (start 81.121798 61.22) (end 77.558298 57.6565) (width 0.635) (layer "F.Cu") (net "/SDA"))
 (segment (start 77.558298 57.6565) (end 62.359034 57.6565) (width 0.635) (layer "F.Cu") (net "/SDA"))
 (segment (start 62.65949 59.84649) (end 65.813 63) (width 0.635) (layer "F.Cu") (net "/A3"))
 (segment (start 52.56501 54.457051) (end 57.954449 59.84649) (width 0.635) (layer "F.Cu") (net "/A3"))
 (segment (start 65.813 63) (end 75 63) (width 0.635) (layer "F.Cu") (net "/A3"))
 (segment (start 57.954449 59.84649) (end 62.65949 59.84649) (width 0.635) (layer "F.Cu") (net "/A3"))
 (segment (start 52.56501 50.5) (end 52.56501 54.457051) (width 0.635) (layer "F.Cu") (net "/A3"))
 (segment (start 79 79.2) (end 79.867 79.2) (width 0.635) (layer "F.Cu") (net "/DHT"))
 (segment (start 53.312045 48.6965) (end 55.10501 50.489465) (width 0.635) (layer "F.Cu") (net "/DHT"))
 (segment (start 79.867 79.2) (end 80.7035 80.0365) (width 0.635) (layer "F.Cu") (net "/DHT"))
 (segment (start 39.65451 52.1835) (end 43.14151 48.6965) (width 0.635) (layer "F.Cu") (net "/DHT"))
 (segment (start 75.343505 88.803495) (end 49.566907 88.803495) (width 0.635) (layer "F.Cu") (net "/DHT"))
 (segment (start 43.14151 48.6965) (end 53.312045 48.6965) (width 0.635) (layer "F.Cu") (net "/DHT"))
 (segment (start 80.7035 80.0365) (end 80.7035 83.4435) (width 0.635) (layer "F.Cu") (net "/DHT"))
 (segment (start 80.7035 83.4435) (end 75.343505 88.803495) (width 0.635) (layer "F.Cu") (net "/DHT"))
 (segment (start 49.566907 88.803495) (end 39.65451 78.891098) (width 0.635) (layer "F.Cu") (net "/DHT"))
 (segment (start 39.65451 78.891098) (end 39.65451 52.1835) (width 0.635) (layer "F.Cu") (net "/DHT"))
 (segment (start 55.10501 50.489465) (end 55.10501 50.5) (width 0.635) (layer "F.Cu") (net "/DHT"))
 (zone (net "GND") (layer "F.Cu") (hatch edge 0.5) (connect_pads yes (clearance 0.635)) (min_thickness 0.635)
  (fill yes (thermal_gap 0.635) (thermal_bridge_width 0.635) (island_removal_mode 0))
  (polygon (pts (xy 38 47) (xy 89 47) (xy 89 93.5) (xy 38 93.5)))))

